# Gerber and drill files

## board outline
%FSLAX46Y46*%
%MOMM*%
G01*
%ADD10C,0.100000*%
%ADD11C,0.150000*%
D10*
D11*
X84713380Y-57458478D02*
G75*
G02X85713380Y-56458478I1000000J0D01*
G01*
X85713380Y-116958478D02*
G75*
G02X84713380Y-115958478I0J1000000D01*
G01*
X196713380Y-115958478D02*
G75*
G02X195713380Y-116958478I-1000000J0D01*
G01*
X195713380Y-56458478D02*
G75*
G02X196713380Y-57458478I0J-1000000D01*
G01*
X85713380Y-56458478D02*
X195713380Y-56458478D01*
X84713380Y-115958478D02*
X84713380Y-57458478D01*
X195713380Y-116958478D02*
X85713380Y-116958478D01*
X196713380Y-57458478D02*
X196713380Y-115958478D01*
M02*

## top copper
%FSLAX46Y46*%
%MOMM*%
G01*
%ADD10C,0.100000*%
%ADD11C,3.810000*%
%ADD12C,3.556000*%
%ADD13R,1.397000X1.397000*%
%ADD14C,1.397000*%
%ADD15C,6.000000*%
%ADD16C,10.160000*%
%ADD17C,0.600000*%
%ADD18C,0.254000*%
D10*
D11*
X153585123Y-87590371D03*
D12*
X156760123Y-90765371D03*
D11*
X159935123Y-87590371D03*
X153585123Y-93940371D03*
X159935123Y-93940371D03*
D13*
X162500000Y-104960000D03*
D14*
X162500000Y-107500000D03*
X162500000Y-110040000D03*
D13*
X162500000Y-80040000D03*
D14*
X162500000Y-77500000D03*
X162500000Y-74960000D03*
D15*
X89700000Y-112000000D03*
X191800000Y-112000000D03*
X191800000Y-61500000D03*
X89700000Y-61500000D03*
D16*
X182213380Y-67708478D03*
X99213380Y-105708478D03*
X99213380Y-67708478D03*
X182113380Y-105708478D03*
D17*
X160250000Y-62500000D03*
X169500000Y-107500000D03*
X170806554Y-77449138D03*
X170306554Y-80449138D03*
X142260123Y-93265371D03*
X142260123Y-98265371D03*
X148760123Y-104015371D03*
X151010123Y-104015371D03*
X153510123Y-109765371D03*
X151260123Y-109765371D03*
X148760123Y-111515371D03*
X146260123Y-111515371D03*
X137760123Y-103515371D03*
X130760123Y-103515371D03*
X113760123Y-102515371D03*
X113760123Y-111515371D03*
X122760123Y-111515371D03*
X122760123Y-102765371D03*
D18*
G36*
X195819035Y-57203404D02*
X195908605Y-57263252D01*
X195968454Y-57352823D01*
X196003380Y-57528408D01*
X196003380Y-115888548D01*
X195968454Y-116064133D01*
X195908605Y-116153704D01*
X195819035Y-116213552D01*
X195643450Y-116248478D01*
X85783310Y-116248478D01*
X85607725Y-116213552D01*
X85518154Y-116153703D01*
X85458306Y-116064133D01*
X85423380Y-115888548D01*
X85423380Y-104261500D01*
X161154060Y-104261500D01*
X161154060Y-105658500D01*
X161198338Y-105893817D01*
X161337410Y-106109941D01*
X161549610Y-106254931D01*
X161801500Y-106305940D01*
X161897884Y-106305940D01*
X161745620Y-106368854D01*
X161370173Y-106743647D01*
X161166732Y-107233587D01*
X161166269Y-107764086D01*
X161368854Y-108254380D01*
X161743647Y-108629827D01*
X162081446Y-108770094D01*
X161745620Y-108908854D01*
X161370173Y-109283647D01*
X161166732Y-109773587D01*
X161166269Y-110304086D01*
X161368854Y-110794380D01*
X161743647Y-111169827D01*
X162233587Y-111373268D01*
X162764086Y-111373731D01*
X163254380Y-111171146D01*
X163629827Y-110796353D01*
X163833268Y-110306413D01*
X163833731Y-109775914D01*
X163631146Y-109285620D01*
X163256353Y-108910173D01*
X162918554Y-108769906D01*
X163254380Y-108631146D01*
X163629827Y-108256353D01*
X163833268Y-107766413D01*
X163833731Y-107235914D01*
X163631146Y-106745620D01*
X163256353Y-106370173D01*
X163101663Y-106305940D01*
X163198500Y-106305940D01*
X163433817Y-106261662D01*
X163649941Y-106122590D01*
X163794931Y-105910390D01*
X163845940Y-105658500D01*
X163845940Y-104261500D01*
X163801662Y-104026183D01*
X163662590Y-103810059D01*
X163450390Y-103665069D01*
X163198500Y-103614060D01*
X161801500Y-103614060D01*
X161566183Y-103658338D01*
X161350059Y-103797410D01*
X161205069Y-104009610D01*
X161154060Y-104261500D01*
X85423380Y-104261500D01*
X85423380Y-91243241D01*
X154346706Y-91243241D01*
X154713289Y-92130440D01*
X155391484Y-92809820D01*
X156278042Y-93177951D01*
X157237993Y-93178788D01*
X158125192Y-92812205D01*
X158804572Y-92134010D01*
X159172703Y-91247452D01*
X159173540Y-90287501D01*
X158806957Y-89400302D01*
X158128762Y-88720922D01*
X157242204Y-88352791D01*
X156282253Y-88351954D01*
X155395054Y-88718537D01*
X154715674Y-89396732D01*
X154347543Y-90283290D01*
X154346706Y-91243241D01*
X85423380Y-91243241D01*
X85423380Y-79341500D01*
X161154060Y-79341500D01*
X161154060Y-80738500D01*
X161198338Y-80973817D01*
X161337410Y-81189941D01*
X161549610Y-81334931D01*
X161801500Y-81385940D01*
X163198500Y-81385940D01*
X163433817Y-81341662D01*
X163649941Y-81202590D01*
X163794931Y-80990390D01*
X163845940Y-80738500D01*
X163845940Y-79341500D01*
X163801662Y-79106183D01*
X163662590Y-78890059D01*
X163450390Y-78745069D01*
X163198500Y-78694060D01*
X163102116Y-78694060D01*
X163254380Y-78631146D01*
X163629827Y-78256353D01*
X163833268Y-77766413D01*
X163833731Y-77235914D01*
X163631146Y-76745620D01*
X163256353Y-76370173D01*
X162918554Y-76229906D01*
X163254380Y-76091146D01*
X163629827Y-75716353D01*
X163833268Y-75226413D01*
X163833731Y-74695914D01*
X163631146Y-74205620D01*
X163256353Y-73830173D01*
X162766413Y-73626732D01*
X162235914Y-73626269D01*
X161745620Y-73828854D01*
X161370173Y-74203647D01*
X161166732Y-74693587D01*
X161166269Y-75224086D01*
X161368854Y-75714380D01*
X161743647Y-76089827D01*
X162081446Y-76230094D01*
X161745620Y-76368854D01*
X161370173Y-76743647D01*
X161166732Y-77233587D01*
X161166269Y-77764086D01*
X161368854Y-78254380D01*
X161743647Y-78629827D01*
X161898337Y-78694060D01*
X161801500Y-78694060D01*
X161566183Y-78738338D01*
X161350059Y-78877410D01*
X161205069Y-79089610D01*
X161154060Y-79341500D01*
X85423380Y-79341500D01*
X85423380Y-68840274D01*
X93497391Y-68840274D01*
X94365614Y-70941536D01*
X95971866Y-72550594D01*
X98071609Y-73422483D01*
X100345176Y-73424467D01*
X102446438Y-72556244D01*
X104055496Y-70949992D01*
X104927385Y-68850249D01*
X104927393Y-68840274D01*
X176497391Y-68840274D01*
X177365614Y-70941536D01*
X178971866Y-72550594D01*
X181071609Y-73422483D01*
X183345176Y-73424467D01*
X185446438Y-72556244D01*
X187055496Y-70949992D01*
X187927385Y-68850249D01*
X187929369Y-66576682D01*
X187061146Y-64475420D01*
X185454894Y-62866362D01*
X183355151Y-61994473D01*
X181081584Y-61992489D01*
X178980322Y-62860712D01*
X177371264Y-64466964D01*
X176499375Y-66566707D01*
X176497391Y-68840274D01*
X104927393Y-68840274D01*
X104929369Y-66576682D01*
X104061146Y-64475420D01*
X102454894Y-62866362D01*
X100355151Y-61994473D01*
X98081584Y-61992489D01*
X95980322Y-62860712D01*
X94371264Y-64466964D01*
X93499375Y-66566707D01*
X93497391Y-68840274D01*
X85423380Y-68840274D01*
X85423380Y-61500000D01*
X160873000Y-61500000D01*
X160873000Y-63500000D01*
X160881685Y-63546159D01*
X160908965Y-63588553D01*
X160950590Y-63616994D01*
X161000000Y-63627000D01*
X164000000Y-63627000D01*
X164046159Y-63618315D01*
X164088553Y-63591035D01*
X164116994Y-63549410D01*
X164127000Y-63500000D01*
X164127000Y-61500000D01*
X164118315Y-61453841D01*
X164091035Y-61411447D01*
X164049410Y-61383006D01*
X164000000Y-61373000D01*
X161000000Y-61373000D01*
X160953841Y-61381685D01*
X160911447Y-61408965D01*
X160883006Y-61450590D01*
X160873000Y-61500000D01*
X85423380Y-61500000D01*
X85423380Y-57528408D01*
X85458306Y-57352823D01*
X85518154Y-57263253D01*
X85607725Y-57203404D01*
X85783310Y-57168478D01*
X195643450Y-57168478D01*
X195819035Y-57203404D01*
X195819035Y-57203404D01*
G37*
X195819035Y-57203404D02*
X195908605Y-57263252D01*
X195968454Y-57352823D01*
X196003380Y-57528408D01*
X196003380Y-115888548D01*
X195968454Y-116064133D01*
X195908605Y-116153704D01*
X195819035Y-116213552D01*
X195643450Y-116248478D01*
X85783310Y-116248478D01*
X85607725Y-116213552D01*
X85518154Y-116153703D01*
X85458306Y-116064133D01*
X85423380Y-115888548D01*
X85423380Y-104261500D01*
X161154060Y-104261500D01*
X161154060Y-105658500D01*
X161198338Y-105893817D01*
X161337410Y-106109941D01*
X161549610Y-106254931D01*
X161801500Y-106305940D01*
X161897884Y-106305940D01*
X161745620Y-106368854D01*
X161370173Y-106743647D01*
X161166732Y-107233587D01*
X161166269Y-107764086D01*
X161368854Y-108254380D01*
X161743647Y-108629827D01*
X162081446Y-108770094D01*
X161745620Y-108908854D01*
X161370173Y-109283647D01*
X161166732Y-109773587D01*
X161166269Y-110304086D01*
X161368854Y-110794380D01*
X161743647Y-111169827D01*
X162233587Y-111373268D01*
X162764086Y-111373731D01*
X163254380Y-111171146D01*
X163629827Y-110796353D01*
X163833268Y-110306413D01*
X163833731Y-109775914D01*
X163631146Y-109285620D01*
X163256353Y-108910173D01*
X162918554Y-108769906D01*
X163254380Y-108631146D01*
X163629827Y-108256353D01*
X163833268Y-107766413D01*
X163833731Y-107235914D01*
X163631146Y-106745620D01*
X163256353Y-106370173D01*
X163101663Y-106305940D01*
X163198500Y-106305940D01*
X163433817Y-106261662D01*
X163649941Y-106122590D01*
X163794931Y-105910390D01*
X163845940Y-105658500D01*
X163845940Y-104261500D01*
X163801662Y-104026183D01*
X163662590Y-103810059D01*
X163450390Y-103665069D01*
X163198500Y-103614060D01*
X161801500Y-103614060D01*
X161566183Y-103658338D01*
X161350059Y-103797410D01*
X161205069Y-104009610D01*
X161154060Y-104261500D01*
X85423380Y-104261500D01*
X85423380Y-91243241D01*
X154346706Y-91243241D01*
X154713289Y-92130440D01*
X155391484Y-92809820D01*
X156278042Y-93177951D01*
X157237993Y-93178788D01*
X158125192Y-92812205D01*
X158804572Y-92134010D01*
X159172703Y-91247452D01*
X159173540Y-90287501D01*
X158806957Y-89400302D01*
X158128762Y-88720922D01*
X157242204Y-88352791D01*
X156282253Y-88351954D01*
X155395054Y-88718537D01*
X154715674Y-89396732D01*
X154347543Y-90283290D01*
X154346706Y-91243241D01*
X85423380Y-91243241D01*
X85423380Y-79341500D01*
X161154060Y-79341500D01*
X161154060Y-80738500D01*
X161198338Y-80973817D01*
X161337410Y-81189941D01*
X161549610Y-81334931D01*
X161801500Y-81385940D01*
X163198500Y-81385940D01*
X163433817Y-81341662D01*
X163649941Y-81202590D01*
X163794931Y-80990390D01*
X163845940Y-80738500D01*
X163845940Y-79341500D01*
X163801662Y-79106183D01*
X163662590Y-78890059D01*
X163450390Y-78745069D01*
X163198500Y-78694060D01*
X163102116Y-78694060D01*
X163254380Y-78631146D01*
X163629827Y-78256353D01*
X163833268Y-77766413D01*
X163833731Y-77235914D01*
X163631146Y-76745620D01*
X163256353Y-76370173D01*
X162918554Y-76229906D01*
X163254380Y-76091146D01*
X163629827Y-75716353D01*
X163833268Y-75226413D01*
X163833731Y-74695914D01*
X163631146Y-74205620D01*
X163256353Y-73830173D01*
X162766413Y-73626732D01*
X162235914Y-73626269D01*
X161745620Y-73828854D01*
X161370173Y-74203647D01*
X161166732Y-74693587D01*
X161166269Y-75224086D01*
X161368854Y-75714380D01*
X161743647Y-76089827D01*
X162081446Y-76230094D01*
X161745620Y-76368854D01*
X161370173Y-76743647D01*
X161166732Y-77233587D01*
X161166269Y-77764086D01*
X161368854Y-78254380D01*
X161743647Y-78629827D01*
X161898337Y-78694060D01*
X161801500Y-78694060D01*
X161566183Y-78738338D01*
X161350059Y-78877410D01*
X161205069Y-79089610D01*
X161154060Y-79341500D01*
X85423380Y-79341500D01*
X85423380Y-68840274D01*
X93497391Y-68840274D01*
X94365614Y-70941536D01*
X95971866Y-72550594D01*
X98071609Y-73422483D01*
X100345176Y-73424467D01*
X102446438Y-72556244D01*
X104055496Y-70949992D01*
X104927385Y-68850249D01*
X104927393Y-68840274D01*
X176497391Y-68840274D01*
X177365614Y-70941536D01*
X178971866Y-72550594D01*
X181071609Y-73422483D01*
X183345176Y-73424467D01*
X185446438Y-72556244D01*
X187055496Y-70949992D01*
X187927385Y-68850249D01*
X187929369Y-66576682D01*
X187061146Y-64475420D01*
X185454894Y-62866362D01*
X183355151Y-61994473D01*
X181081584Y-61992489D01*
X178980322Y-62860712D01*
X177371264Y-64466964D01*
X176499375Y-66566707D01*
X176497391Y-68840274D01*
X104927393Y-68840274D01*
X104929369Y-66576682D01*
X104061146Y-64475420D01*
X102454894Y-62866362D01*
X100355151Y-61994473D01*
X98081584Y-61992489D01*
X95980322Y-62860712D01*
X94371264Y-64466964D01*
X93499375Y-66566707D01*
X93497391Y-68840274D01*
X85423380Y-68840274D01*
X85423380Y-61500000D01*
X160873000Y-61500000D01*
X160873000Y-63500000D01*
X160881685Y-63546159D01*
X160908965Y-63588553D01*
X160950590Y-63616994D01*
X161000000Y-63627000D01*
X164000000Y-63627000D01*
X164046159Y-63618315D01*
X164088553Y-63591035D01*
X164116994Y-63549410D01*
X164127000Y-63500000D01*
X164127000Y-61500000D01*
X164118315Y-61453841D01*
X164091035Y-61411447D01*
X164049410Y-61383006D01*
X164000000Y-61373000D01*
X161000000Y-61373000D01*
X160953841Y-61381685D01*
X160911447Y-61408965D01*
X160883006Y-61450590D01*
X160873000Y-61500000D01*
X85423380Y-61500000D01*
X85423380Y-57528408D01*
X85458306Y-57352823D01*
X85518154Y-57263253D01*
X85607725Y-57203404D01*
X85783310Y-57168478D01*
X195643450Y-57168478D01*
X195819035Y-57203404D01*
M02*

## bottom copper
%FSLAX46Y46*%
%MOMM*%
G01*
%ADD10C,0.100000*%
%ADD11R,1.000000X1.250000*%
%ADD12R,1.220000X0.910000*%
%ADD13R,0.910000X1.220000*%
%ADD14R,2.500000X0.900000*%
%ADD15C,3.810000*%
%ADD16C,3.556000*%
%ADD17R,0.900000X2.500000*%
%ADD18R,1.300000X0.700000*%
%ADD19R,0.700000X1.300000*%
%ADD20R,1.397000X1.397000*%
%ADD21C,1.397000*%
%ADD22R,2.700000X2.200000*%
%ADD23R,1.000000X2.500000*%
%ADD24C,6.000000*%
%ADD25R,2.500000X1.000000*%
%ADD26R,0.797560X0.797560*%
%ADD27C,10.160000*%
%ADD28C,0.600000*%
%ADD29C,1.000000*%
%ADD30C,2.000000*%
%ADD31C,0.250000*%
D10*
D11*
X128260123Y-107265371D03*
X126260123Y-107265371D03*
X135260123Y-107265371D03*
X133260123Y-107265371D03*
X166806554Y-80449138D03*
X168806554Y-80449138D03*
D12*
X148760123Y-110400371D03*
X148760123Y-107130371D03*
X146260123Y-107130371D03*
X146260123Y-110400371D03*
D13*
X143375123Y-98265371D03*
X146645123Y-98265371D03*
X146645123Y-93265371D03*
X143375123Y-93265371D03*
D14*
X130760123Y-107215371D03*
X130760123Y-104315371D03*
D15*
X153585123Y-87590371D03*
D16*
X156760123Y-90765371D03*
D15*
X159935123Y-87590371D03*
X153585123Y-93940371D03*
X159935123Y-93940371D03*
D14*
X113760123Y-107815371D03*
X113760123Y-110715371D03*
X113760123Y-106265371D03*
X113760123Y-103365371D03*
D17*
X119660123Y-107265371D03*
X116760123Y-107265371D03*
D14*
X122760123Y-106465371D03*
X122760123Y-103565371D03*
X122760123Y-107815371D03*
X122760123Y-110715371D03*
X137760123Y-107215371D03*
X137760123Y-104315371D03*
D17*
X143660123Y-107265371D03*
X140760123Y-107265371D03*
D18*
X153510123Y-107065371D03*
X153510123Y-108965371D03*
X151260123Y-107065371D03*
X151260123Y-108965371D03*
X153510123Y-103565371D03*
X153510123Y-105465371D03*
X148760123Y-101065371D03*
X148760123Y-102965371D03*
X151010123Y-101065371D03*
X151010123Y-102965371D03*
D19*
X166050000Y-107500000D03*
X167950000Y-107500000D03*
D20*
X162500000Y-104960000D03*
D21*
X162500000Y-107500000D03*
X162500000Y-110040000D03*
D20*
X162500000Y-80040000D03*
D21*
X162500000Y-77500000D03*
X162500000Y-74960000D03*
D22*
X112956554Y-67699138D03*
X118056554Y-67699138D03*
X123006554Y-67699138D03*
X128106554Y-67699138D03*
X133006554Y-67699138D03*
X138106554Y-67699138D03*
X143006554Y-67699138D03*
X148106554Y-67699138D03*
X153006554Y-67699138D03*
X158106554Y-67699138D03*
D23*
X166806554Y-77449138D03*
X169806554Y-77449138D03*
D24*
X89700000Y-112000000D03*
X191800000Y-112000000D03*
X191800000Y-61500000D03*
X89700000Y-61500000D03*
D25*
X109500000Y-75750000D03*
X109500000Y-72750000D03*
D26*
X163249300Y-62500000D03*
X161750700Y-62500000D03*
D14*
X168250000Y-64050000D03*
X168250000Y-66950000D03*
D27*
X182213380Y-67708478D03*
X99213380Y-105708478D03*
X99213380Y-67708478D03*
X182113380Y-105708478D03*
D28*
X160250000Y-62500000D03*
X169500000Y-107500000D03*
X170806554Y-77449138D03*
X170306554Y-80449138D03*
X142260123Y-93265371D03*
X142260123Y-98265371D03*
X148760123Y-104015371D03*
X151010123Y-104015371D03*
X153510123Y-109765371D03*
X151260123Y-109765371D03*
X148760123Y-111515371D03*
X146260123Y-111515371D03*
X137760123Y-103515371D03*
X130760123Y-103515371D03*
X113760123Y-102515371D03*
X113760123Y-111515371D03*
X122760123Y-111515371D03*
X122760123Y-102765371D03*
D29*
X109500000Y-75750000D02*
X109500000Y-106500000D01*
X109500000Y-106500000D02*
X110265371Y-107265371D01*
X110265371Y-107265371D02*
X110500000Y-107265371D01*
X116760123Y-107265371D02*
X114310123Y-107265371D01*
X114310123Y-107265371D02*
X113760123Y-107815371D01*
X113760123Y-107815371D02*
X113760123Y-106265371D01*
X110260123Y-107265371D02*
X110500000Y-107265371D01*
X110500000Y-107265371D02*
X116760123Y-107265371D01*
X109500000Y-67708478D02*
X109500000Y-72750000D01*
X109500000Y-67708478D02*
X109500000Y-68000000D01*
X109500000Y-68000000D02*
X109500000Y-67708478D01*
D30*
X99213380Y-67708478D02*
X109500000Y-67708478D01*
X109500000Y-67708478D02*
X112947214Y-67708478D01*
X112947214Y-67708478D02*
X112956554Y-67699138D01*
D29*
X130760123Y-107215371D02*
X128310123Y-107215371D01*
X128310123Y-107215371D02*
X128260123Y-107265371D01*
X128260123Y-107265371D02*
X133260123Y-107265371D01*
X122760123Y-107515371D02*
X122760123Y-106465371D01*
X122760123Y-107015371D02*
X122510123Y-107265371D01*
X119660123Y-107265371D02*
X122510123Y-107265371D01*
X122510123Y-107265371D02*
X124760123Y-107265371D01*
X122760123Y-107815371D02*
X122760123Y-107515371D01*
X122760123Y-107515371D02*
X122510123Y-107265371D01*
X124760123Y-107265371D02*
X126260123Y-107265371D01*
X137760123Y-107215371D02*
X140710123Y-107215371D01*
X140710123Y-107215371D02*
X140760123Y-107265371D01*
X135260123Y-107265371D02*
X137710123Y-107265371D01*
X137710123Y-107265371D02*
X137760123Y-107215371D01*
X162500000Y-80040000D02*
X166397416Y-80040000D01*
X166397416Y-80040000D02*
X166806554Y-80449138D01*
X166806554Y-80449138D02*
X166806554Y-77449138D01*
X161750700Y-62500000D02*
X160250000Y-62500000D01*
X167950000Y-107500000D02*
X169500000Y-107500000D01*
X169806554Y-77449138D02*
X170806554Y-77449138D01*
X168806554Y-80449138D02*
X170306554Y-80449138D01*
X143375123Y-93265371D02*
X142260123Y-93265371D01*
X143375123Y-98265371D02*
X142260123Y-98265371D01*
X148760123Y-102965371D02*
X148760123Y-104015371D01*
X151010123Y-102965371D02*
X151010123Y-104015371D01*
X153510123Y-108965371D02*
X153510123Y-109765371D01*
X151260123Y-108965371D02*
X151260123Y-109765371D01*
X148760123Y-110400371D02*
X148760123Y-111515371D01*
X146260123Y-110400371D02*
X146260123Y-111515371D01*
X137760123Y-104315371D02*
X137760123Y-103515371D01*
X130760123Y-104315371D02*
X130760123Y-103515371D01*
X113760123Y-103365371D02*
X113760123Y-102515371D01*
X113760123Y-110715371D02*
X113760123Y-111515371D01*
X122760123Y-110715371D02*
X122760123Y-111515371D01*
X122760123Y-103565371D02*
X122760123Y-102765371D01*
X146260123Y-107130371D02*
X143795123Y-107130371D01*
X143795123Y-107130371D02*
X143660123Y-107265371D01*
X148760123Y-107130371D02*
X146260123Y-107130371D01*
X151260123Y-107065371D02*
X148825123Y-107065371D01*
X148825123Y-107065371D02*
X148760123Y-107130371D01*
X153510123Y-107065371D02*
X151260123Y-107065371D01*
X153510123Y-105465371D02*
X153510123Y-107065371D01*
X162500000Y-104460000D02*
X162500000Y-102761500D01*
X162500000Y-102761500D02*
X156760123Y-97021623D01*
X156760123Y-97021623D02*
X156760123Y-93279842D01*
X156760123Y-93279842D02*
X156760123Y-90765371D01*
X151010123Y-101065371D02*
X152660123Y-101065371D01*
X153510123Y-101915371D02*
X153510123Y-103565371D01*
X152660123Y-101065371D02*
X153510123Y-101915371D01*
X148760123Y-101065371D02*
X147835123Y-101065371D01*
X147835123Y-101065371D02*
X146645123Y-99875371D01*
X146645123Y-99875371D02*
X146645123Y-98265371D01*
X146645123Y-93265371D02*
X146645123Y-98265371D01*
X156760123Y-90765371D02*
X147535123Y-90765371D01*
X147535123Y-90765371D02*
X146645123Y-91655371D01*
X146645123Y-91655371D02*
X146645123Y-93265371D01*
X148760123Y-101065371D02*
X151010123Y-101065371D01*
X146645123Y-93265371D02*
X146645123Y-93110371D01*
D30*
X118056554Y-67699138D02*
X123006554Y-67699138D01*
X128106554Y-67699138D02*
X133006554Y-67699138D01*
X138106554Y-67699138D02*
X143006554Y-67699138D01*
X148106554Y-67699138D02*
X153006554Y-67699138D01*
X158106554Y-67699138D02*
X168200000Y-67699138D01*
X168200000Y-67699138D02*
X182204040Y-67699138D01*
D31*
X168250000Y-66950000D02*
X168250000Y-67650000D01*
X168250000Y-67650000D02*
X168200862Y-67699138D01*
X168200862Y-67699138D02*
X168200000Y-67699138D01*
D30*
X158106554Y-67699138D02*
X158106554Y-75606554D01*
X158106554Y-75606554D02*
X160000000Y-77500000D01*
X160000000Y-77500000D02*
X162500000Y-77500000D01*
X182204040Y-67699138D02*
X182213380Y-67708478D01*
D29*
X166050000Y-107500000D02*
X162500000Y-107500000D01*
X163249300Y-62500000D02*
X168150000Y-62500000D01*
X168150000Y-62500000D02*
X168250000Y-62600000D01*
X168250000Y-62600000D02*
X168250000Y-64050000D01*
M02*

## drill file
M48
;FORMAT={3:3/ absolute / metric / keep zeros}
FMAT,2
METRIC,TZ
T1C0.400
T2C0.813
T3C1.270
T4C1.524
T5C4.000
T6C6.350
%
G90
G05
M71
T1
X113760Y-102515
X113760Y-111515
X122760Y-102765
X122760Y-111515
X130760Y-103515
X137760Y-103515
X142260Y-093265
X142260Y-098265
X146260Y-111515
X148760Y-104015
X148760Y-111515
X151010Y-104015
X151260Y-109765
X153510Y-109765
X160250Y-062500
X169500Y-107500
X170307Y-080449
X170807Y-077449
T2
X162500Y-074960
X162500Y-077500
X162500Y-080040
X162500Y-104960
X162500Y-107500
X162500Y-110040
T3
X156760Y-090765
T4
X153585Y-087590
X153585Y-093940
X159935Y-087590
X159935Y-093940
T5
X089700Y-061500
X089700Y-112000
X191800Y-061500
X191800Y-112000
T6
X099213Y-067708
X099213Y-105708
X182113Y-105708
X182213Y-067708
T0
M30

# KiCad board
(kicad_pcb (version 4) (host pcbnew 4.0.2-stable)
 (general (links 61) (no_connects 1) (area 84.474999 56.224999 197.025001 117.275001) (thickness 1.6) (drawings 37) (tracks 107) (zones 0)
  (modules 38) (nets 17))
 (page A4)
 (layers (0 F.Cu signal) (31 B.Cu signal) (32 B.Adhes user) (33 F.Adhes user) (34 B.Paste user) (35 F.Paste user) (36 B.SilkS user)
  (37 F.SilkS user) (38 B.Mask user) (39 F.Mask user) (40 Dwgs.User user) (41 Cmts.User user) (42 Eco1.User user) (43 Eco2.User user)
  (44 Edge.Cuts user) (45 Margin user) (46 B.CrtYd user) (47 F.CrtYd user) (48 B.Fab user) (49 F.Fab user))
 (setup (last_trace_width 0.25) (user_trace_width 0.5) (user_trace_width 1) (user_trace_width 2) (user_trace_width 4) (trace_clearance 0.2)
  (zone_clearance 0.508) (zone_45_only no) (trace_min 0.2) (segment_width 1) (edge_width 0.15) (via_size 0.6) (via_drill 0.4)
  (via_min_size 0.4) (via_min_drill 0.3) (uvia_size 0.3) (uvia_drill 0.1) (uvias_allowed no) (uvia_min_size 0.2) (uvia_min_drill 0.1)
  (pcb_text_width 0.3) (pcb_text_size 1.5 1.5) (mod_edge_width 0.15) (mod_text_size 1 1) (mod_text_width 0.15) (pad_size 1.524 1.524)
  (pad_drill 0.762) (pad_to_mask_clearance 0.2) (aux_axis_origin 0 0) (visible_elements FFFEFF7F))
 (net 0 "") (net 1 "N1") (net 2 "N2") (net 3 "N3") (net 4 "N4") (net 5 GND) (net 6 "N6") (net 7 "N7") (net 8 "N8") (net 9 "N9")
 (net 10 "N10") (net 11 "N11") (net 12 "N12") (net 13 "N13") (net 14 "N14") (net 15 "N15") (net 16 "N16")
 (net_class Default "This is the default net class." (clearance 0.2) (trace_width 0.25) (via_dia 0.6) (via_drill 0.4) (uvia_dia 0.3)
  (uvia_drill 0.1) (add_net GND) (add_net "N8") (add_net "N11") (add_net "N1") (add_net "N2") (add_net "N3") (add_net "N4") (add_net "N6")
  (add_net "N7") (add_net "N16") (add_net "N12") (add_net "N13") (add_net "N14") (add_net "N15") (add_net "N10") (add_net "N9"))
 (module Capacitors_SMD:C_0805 (layer B.Cu) (at 127.260123 107.265371 180)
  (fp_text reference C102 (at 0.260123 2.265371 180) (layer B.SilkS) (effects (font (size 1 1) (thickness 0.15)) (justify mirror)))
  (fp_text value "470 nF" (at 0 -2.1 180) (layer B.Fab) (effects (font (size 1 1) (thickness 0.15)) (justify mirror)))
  (pad 1 smd rect (at -1 0 180) (size 1 1.25) (layers B.Cu B.Paste B.Mask) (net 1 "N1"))
  (pad 2 smd rect (at 1 0 180) (size 1 1.25) (layers B.Cu B.Paste B.Mask) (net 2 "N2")))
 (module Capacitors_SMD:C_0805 (layer B.Cu) (at 134.260123 107.265371 180)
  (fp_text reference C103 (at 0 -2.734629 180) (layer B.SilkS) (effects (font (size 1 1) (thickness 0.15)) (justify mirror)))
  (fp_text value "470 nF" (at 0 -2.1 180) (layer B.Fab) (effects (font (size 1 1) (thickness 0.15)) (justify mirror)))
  (pad 1 smd rect (at -1 0 180) (size 1 1.25) (layers B.Cu B.Paste B.Mask) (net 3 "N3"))
  (pad 2 smd rect (at 1 0 180) (size 1 1.25) (layers B.Cu B.Paste B.Mask) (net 1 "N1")))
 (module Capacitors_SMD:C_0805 (layer B.Cu) (at 167.806554 80.449138)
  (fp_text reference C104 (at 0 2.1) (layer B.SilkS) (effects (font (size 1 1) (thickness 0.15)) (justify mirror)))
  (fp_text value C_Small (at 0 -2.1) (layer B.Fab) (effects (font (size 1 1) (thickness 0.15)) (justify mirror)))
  (pad 1 smd rect (at -1 0) (size 1 1.25) (layers B.Cu B.Paste B.Mask) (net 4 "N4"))
  (pad 2 smd rect (at 1 0) (size 1 1.25) (layers B.Cu B.Paste B.Mask) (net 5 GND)))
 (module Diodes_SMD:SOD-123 (layer B.Cu) (at 148.760123 108.765371 90)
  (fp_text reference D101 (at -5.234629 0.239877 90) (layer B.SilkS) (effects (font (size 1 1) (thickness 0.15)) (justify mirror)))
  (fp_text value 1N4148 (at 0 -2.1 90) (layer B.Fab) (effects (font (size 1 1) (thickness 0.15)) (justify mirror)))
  (pad 1 smd rect (at -1.635 0 90) (size 0.91 1.22) (layers B.Cu B.Paste B.Mask) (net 5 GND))
  (pad 2 smd rect (at 1.635 0 90) (size 0.91 1.22) (layers B.Cu B.Paste B.Mask) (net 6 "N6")))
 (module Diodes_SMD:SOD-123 (layer B.Cu) (at 146.260123 108.765371 270)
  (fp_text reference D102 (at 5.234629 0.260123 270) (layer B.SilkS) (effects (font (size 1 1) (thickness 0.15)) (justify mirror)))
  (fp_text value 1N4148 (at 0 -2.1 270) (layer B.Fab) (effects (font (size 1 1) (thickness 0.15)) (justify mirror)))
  (pad 1 smd rect (at -1.635 0 270) (size 0.91 1.22) (layers B.Cu B.Paste B.Mask) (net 6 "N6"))
  (pad 2 smd rect (at 1.635 0 270) (size 0.91 1.22) (layers B.Cu B.Paste B.Mask) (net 5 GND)))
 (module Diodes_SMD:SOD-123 (layer B.Cu) (at 145.010123 98.265371)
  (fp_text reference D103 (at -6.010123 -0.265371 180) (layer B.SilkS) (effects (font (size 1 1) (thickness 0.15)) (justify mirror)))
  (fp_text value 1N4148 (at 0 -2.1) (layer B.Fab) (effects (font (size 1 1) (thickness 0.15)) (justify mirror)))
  (pad 1 smd rect (at -1.635 0) (size 0.91 1.22) (layers B.Cu B.Paste B.Mask) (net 5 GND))
  (pad 2 smd rect (at 1.635 0) (size 0.91 1.22) (layers B.Cu B.Paste B.Mask) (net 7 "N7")))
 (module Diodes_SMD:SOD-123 (layer B.Cu) (at 145.010123 93.265371 180)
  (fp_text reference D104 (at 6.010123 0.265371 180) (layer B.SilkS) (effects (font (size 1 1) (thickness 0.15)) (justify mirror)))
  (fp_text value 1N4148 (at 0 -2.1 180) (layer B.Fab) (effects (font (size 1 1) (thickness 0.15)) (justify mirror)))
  (pad 1 smd rect (at -1.635 0 180) (size 0.91 1.22) (layers B.Cu B.Paste B.Mask) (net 7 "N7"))
  (pad 2 smd rect (at 1.635 0 180) (size 0.91 1.22) (layers B.Cu B.Paste B.Mask) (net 5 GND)))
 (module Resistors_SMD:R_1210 (layer B.Cu) (at 130.760123 105.765371 90)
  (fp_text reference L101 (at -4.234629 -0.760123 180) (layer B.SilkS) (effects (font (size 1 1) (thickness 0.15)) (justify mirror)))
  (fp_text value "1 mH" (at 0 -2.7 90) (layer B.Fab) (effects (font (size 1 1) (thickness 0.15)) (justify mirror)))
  (pad 1 smd rect (at -1.45 0 90) (size 0.9 2.5) (layers B.Cu B.Paste B.Mask) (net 1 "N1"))
  (pad 2 smd rect (at 1.45 0 90) (size 0.9 2.5) (layers B.Cu B.Paste B.Mask) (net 5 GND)))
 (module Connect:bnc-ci (layer F.Cu) (at 156.760123 90.765371)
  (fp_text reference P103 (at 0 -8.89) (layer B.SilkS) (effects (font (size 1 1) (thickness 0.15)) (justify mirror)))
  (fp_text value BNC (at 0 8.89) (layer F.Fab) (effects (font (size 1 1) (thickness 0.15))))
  (pad 2 thru_hole circle (at -3.175 -3.175) (size 3.81 3.81) (drill 1.524) (layers *.Cu *.Mask F.SilkS) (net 5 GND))
  (pad 1 thru_hole circle (at 0 0) (size 3.556 3.556) (drill 1.27) (layers *.Cu *.Mask F.SilkS) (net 7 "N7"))
  (pad 2 thru_hole circle (at 3.175 -3.175) (size 3.81 3.81) (drill 1.524) (layers *.Cu *.Mask F.SilkS) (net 5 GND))
  (pad 2 thru_hole circle (at -3.175 3.175) (size 3.81 3.81) (drill 1.524) (layers *.Cu *.Mask F.SilkS) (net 5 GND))
  (pad 2 thru_hole circle (at 3.175 3.175) (size 3.81 3.81) (drill 1.524) (layers *.Cu *.Mask F.SilkS) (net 5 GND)))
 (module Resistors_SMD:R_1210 (layer B.Cu) (at 113.760123 109.265371 270)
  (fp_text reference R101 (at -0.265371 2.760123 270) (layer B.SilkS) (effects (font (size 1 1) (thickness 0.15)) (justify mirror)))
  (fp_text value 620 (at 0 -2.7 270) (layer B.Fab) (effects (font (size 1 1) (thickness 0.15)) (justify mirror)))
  (pad 1 smd rect (at -1.45 0 270) (size 0.9 2.5) (layers B.Cu B.Paste B.Mask) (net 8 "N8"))
  (pad 2 smd rect (at 1.45 0 270) (size 0.9 2.5) (layers B.Cu B.Paste B.Mask) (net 5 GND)))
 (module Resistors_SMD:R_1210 (layer B.Cu) (at 113.760123 104.815371 90)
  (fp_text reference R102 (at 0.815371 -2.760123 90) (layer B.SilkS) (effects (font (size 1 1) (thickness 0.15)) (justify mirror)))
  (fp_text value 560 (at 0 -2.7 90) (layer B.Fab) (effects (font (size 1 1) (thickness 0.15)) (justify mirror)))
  (pad 1 smd rect (at -1.45 0 90) (size 0.9 2.5) (layers B.Cu B.Paste B.Mask) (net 8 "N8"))
  (pad 2 smd rect (at 1.45 0 90) (size 0.9 2.5) (layers B.Cu B.Paste B.Mask) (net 5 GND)))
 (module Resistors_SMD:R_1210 (layer B.Cu) (at 118.210123 107.265371 180)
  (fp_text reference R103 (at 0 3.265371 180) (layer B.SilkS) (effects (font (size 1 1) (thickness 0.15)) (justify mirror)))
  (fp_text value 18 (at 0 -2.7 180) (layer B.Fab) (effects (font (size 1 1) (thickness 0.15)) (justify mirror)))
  (pad 1 smd rect (at -1.45 0 180) (size 0.9 2.5) (layers B.Cu B.Paste B.Mask) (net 2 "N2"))
  (pad 2 smd rect (at 1.45 0 180) (size 0.9 2.5) (layers B.Cu B.Paste B.Mask) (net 8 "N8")))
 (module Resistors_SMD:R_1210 (layer B.Cu) (at 122.760123 105.015371 90)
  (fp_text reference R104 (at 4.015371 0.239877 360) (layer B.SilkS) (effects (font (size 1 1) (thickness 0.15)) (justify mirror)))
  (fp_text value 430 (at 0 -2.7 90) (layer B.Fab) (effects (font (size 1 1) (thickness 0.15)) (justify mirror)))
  (pad 1 smd rect (at -1.45 0 90) (size 0.9 2.5) (layers B.Cu B.Paste B.Mask) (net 2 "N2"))
  (pad 2 smd rect (at 1.45 0 90) (size 0.9 2.5) (layers B.Cu B.Paste B.Mask) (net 5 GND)))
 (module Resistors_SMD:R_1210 (layer B.Cu) (at 122.760123 109.265371 270)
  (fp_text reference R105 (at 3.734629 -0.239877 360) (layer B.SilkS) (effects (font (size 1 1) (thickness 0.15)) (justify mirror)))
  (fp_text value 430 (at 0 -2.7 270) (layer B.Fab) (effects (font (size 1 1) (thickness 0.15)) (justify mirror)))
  (pad 1 smd rect (at -1.45 0 270) (size 0.9 2.5) (layers B.Cu B.Paste B.Mask) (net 2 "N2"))
  (pad 2 smd rect (at 1.45 0 270) (size 0.9 2.5) (layers B.Cu B.Paste B.Mask) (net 5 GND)))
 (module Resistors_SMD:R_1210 (layer B.Cu) (at 137.760123 105.765371 90)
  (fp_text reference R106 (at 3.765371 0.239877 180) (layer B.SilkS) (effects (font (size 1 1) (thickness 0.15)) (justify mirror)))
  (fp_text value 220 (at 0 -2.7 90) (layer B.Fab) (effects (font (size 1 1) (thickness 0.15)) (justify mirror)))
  (pad 1 smd rect (at -1.45 0 90) (size 0.9 2.5) (layers B.Cu B.Paste B.Mask) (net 3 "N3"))
  (pad 2 smd rect (at 1.45 0 90) (size 0.9 2.5) (layers B.Cu B.Paste B.Mask) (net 5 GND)))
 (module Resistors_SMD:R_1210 (layer B.Cu) (at 142.210123 107.265371 180)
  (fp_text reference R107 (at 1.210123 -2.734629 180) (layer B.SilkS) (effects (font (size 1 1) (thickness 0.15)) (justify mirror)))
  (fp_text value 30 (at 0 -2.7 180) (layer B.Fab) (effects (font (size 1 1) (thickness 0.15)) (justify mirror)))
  (pad 1 smd rect (at -1.45 0 180) (size 0.9 2.5) (layers B.Cu B.Paste B.Mask) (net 6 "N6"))
  (pad 2 smd rect (at 1.45 0 180) (size 0.9 2.5) (layers B.Cu B.Paste B.Mask) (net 3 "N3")))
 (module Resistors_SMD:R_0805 (layer B.Cu) (at 153.510123 108.015371 270)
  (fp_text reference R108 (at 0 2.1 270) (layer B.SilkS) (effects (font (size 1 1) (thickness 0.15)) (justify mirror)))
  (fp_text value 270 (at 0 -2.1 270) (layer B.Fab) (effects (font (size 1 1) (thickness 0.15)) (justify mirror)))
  (pad 1 smd rect (at -0.95 0 270) (size 0.7 1.3) (layers B.Cu B.Paste B.Mask) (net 6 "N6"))
  (pad 2 smd rect (at 0.95 0 270) (size 0.7 1.3) (layers B.Cu B.Paste B.Mask) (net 5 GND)))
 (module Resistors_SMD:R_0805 (layer B.Cu) (at 151.260123 108.015371 270)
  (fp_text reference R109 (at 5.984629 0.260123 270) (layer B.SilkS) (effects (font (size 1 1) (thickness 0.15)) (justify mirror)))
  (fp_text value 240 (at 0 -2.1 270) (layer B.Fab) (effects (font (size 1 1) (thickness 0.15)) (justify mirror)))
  (pad 1 smd rect (at -0.95 0 270) (size 0.7 1.3) (layers B.Cu B.Paste B.Mask) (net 6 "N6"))
  (pad 2 smd rect (at 0.95 0 270) (size 0.7 1.3) (layers B.Cu B.Paste B.Mask) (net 5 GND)))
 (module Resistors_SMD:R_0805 (layer B.Cu) (at 153.510123 104.515371 270)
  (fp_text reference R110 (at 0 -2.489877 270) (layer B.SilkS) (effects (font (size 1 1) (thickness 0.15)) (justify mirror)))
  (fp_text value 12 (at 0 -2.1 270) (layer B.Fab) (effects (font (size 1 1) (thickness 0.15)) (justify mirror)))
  (pad 1 smd rect (at -0.95 0 270) (size 0.7 1.3) (layers B.Cu B.Paste B.Mask) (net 7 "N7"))
  (pad 2 smd rect (at 0.95 0 270) (size 0.7 1.3) (layers B.Cu B.Paste B.Mask) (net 6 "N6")))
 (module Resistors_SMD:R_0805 (layer B.Cu) (at 148.760123 102.015371 270)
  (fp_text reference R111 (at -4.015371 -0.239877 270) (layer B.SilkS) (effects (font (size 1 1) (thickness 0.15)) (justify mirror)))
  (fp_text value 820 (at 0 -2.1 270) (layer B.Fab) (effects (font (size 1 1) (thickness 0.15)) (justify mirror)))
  (pad 1 smd rect (at -0.95 0 270) (size 0.7 1.3) (layers B.Cu B.Paste B.Mask) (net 7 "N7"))
  (pad 2 smd rect (at 0.95 0 270) (size 0.7 1.3) (layers B.Cu B.Paste B.Mask) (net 5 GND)))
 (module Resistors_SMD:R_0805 (layer B.Cu) (at 151.010123 102.015371 270)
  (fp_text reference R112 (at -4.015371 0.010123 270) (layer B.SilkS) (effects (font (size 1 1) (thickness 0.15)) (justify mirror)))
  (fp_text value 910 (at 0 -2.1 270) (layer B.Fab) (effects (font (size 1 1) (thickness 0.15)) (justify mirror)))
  (pad 1 smd rect (at -0.95 0 270) (size 0.7 1.3) (layers B.Cu B.Paste B.Mask) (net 7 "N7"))
  (pad 2 smd rect (at 0.95 0 270) (size 0.7 1.3) (layers B.Cu B.Paste B.Mask) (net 5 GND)))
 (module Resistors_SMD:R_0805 (layer B.Cu) (at 167 107.5)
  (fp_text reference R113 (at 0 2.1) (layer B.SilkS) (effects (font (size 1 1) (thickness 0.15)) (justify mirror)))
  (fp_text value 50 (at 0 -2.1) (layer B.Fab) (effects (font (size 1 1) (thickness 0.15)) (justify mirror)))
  (pad 1 smd rect (at -0.95 0) (size 0.7 1.3) (layers B.Cu B.Paste B.Mask) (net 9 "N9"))
  (pad 2 smd rect (at 0.95 0) (size 0.7 1.3) (layers B.Cu B.Paste B.Mask) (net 5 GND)))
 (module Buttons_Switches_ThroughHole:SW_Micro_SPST (layer F.Cu) (at 162.5 107.5 270)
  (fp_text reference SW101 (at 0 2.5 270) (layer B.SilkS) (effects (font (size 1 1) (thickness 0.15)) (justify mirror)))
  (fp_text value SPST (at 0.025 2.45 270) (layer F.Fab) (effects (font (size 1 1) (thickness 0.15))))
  (pad 1 thru_hole rect (at -2.54 0 270) (size 1.397 1.397) (drill 0.8128) (layers *.Cu *.Mask F.SilkS) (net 7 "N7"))
  (pad 2 thru_hole circle (at 0 0 270) (size 1.397 1.397) (drill 0.8128) (layers *.Cu *.Mask F.SilkS) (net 9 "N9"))
  (pad 3 thru_hole circle (at 2.54 0 270) (size 1.397 1.397) (drill 0.8128) (layers *.Cu *.Mask F.SilkS)))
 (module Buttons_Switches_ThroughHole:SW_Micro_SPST (layer F.Cu) (at 162.5 77.5 90)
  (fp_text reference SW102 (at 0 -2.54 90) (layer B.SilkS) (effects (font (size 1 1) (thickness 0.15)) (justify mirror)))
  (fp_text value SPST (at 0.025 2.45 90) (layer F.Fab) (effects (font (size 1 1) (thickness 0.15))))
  (pad 1 thru_hole rect (at -2.54 0 90) (size 1.397 1.397) (drill 0.8128) (layers *.Cu *.Mask F.SilkS) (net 4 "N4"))
  (pad 2 thru_hole circle (at 0 0 90) (size 1.397 1.397) (drill 0.8128) (layers *.Cu *.Mask F.SilkS) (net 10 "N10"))
  (pad 3 thru_hole circle (at 2.54 0 90) (size 1.397 1.397) (drill 0.8128) (layers *.Cu *.Mask F.SilkS)))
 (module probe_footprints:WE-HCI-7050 (layer B.Cu) (at 115.506554 67.699138)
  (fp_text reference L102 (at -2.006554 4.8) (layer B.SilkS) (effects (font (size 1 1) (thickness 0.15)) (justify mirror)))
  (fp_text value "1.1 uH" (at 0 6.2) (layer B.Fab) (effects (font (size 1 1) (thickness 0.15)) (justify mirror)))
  (pad 1 smd rect (at -2.55 0) (size 2.7 2.2) (layers B.Cu B.Paste B.Mask) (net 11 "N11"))
  (pad 2 smd rect (at 2.55 0) (size 2.7 2.2) (layers B.Cu B.Paste B.Mask) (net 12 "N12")))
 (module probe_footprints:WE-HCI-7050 (layer B.Cu) (at 125.556554 67.699138)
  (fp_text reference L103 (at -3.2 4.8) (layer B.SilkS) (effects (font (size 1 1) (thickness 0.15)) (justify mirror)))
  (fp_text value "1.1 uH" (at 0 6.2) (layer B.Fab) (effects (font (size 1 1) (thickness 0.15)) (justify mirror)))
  (pad 1 smd rect (at -2.55 0) (size 2.7 2.2) (layers B.Cu B.Paste B.Mask) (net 12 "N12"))
  (pad 2 smd rect (at 2.55 0) (size 2.7 2.2) (layers B.Cu B.Paste B.Mask) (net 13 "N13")))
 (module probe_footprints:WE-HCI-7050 (layer B.Cu) (at 135.556554 67.699138)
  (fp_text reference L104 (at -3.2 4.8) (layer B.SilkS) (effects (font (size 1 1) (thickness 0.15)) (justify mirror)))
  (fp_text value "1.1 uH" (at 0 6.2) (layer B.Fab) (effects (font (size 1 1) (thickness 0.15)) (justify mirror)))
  (pad 1 smd rect (at -2.55 0) (size 2.7 2.2) (layers B.Cu B.Paste B.Mask) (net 13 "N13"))
  (pad 2 smd rect (at 2.55 0) (size 2.7 2.2) (layers B.Cu B.Paste B.Mask) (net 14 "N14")))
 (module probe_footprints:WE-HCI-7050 (layer B.Cu) (at 145.556554 67.699138)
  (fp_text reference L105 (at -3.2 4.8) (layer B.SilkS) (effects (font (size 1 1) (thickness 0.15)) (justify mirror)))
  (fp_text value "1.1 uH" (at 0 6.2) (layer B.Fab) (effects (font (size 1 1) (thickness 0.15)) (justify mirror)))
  (pad 1 smd rect (at -2.55 0) (size 2.7 2.2) (layers B.Cu B.Paste B.Mask) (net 14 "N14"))
  (pad 2 smd rect (at 2.55 0) (size 2.7 2.2) (layers B.Cu B.Paste B.Mask) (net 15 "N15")))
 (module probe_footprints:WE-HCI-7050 (layer B.Cu) (at 155.556554 67.699138)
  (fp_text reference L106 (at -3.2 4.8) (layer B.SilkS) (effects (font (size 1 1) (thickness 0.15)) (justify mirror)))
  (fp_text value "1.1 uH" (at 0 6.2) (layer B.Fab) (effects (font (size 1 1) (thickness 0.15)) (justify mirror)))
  (pad 1 smd rect (at -2.55 0) (size 2.7 2.2) (layers B.Cu B.Paste B.Mask) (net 15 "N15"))
  (pad 2 smd rect (at 2.55 0) (size 2.7 2.2) (layers B.Cu B.Paste B.Mask) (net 10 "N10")))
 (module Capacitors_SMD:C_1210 (layer B.Cu) (at 168.306554 77.449138)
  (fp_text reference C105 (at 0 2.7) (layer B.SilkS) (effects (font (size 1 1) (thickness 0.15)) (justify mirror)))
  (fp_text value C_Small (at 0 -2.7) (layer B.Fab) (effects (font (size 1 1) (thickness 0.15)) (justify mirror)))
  (pad 1 smd rect (at -1.5 0) (size 1 2.5) (layers B.Cu B.Paste B.Mask) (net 4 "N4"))
  (pad 2 smd rect (at 1.5 0) (size 1 2.5) (layers B.Cu B.Paste B.Mask) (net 5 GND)))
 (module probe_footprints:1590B (layer B.Cu) (at 140.75 86.75 180)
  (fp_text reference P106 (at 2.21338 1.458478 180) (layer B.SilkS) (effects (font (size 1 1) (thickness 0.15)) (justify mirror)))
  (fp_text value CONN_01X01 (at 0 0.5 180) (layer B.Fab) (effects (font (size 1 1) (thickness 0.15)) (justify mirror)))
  (pad 1 thru_hole circle (at 51.05 -25.25 180) (size 6 6) (drill 4) (layers *.Cu *.Mask B.SilkS) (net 5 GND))
  (pad 1 thru_hole circle (at -51.05 -25.25 180) (size 6 6) (drill 4) (layers *.Cu *.Mask B.SilkS) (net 5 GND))
  (pad 1 thru_hole circle (at -51.05 25.25 180) (size 6 6) (drill 4) (layers *.Cu *.Mask B.SilkS) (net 5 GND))
  (pad 1 thru_hole circle (at 51.05 25.25 180) (size 6 6) (drill 4) (layers *.Cu *.Mask B.SilkS) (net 5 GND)))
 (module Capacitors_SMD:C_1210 (layer B.Cu) (at 109.5 74.25 90)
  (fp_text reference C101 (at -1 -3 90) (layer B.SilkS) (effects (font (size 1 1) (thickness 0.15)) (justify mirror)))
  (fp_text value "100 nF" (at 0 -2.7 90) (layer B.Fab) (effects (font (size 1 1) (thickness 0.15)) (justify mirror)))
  (pad 1 smd rect (at -1.5 0 90) (size 1 2.5) (layers B.Cu B.Paste B.Mask) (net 8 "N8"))
  (pad 2 smd rect (at 1.5 0 90) (size 1 2.5) (layers B.Cu B.Paste B.Mask) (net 11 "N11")))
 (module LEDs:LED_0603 (layer B.Cu) (at 162.5 62.5)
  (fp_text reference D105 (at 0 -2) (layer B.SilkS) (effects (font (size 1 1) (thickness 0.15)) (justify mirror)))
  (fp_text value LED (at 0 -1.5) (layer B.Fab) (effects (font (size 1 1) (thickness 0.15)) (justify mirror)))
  (pad 2 smd rect (at 0.7493 0 180) (size 0.79756 0.79756) (layers B.Cu B.Paste B.Mask) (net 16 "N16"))
  (pad 1 smd rect (at -0.7493 0 180) (size 0.79756 0.79756) (layers B.Cu B.Paste B.Mask) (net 5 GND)))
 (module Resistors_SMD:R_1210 (layer B.Cu) (at 168.25 65.5 270)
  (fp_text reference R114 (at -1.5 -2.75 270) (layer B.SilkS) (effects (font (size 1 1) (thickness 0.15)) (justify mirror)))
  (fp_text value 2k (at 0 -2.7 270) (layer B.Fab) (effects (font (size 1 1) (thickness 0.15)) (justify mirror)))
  (pad 1 smd rect (at -1.45 0 270) (size 0.9 2.5) (layers B.Cu B.Paste B.Mask) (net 16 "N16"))
  (pad 2 smd rect (at 1.45 0 270) (size 0.9 2.5) (layers B.Cu B.Paste B.Mask) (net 10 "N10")))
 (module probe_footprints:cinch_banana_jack (layer F.Cu) (at 182.21338 67.708478 270)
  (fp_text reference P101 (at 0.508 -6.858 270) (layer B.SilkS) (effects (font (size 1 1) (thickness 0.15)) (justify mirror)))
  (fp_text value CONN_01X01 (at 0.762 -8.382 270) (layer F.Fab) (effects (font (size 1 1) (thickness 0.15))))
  (pad 1 thru_hole circle (at 0 0 270) (size 10.16 10.16) (drill 6.35) (layers *.Cu *.Mask F.SilkS) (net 10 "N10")))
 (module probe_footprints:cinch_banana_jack (layer F.Cu) (at 99.21338 105.708478 270)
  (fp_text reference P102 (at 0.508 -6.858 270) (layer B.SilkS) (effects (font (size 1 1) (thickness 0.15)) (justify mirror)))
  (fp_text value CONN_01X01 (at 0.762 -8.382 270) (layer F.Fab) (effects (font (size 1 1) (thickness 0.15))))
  (pad 1 thru_hole circle (at 0 0 270) (size 10.16 10.16) (drill 6.35) (layers *.Cu *.Mask F.SilkS) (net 5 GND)))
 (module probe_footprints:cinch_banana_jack (layer F.Cu) (at 99.21338 67.708478 180)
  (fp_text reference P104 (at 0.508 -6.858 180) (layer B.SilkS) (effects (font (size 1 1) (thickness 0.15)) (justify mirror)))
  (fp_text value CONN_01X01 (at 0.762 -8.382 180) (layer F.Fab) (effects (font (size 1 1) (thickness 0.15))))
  (pad 1 thru_hole circle (at 0 0 180) (size 10.16 10.16) (drill 6.35) (layers *.Cu *.Mask F.SilkS) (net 11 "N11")))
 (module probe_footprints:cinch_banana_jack (layer F.Cu) (at 182.11338 105.708478 180)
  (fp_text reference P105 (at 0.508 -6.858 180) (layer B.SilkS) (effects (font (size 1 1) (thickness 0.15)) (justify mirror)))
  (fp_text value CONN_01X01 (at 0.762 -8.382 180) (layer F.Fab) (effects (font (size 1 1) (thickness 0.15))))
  (pad 1 thru_hole circle (at 0 0 180) (size 10.16 10.16) (drill 6.35) (layers *.Cu *.Mask F.SilkS) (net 5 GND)))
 (gr_arc (start 85.71338 57.458478) (end 85.71338 56.458478) (angle -90) (layer Edge.Cuts) (width 0.15))
 (gr_arc (start 85.71338 115.958478) (end 84.71338 115.958478) (angle -90) (layer Edge.Cuts) (width 0.15))
 (gr_arc (start 195.71338 115.958478) (end 195.71338 116.958478) (angle -90) (layer Edge.Cuts) (width 0.15))
 (gr_arc (start 195.71338 57.458478) (end 196.71338 57.458478) (angle -90) (layer Edge.Cuts) (width 0.15))
 (gr_line (start 85.71338 56.458478) (end 195.71338 56.458478) (layer Edge.Cuts) (width 0.15))
 (gr_line (start 84.71338 115.958478) (end 84.71338 57.458478) (layer Edge.Cuts) (width 0.15))
 (gr_line (start 195.71338 116.958478) (end 85.71338 116.958478) (layer Edge.Cuts) (width 0.15))
 (gr_line (start 196.71338 57.458478) (end 196.71338 115.958478) (layer Edge.Cuts) (width 0.15))
 (segment (start 109.5 75.75) (end 109.5 106.5) (width 1) (layer B.Cu) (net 8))
 (segment (start 109.5 106.5) (end 110.265371 107.265371) (width 1) (layer B.Cu) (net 8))
 (segment (start 110.265371 107.265371) (end 110.5 107.265371) (width 1) (layer B.Cu) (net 8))
 (segment (start 116.760123 107.265371) (end 114.310123 107.265371) (width 1) (layer B.Cu) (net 8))
 (segment (start 114.310123 107.265371) (end 113.760123 107.815371) (width 1) (layer B.Cu) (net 8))
 (segment (start 113.760123 107.815371) (end 113.760123 106.265371) (width 1) (layer B.Cu) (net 8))
 (segment (start 110.260123 107.265371) (end 110.5 107.265371) (width 1) (layer B.Cu) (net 8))
 (segment (start 110.5 107.265371) (end 116.760123 107.265371) (width 1) (layer B.Cu) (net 8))
 (segment (start 109.5 67.708478) (end 109.5 72.75) (width 1) (layer B.Cu) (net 11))
 (segment (start 109.5 67.708478) (end 109.5 68) (width 1) (layer B.Cu) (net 11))
 (segment (start 109.5 68) (end 109.5 67.708478) (width 1) (layer B.Cu) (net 11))
 (segment (start 99.21338 67.708478) (end 109.5 67.708478) (width 2) (layer B.Cu) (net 11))
 (segment (start 109.5 67.708478) (end 112.947214 67.708478) (width 2) (layer B.Cu) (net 11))
 (segment (start 112.947214 67.708478) (end 112.956554 67.699138) (width 2) (layer B.Cu) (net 11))
 (segment (start 130.760123 107.215371) (end 128.310123 107.215371) (width 1) (layer B.Cu) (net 1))
 (segment (start 128.310123 107.215371) (end 128.260123 107.265371) (width 1) (layer B.Cu) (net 1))
 (segment (start 128.260123 107.265371) (end 133.260123 107.265371) (width 1) (layer B.Cu) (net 1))
 (segment (start 122.760123 107.515371) (end 122.760123 106.465371) (width 1) (layer B.Cu) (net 2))
 (segment (start 122.760123 107.015371) (end 122.510123 107.265371) (width 1) (layer B.Cu) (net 2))
 (segment (start 119.660123 107.265371) (end 122.510123 107.265371) (width 1) (layer B.Cu) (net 2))
 (segment (start 122.510123 107.265371) (end 124.760123 107.265371) (width 1) (layer B.Cu) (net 2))
 (segment (start 122.760123 107.815371) (end 122.760123 107.515371) (width 1) (layer B.Cu) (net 2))
 (segment (start 122.760123 107.515371) (end 122.510123 107.265371) (width 1) (layer B.Cu) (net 2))
 (segment (start 124.760123 107.265371) (end 126.260123 107.265371) (width 1) (layer B.Cu) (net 2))
 (segment (start 137.760123 107.215371) (end 140.710123 107.215371) (width 1) (layer B.Cu) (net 3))
 (segment (start 140.710123 107.215371) (end 140.760123 107.265371) (width 1) (layer B.Cu) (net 3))
 (segment (start 135.260123 107.265371) (end 137.710123 107.265371) (width 1) (layer B.Cu) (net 3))
 (segment (start 137.710123 107.265371) (end 137.760123 107.215371) (width 1) (layer B.Cu) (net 3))
 (segment (start 162.5 80.04) (end 166.397416 80.04) (width 1) (layer B.Cu) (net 4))
 (segment (start 166.397416 80.04) (end 166.806554 80.449138) (width 1) (layer B.Cu) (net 4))
 (segment (start 166.806554 80.449138) (end 166.806554 77.449138) (width 1) (layer B.Cu) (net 4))
 (via (at 160.25 62.5) (size 0.6) (drill 0.4) (layers F.Cu B.Cu) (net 5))
 (segment (start 161.7507 62.5) (end 160.25 62.5) (width 1) (layer B.Cu) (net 5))
 (segment (start 167.95 107.5) (end 169.5 107.5) (width 1) (layer B.Cu) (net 5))
 (via (at 169.5 107.5) (size 0.6) (drill 0.4) (layers F.Cu B.Cu) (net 5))
 (via (at 170.806554 77.449138) (size 0.6) (drill 0.4) (layers F.Cu B.Cu) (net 5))
 (segment (start 169.806554 77.449138) (end 170.806554 77.449138) (width 1) (layer B.Cu) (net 5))
 (via (at 170.306554 80.449138) (size 0.6) (drill 0.4) (layers F.Cu B.Cu) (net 5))
 (segment (start 168.806554 80.449138) (end 170.306554 80.449138) (width 1) (layer B.Cu) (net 5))
 (via (at 142.260123 93.265371) (size 0.6) (drill 0.4) (layers F.Cu B.Cu) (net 5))
 (segment (start 143.375123 93.265371) (end 142.260123 93.265371) (width 1) (layer B.Cu) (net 5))
 (via (at 142.260123 98.265371) (size 0.6) (drill 0.4) (layers F.Cu B.Cu) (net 5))
 (segment (start 143.375123 98.265371) (end 142.260123 98.265371) (width 1) (layer B.Cu) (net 5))
 (via (at 148.760123 104.015371) (size 0.6) (drill 0.4) (layers F.Cu B.Cu) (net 5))
 (segment (start 148.760123 102.965371) (end 148.760123 104.015371) (width 1) (layer B.Cu) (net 5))
 (via (at 151.010123 104.015371) (size 0.6) (drill 0.4) (layers F.Cu B.Cu) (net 5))
 (segment (start 151.010123 102.965371) (end 151.010123 104.015371) (width 1) (layer B.Cu) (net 5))
 (via (at 153.510123 109.765371) (size 0.6) (drill 0.4) (layers F.Cu B.Cu) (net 5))
 (segment (start 153.510123 108.965371) (end 153.510123 109.765371) (width 1) (layer B.Cu) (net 5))
 (via (at 151.260123 109.765371) (size 0.6) (drill 0.4) (layers F.Cu B.Cu) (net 5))
 (segment (start 151.260123 108.965371) (end 151.260123 109.765371) (width 1) (layer B.Cu) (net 5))
 (via (at 148.760123 111.515371) (size 0.6) (drill 0.4) (layers F.Cu B.Cu) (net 5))
 (segment (start 148.760123 110.400371) (end 148.760123 111.515371) (width 1) (layer B.Cu) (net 5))
 (via (at 146.260123 111.515371) (size 0.6) (drill 0.4) (layers F.Cu B.Cu) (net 5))
 (segment (start 146.260123 110.400371) (end 146.260123 111.515371) (width 1) (layer B.Cu) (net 5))
 (via (at 137.760123 103.515371) (size 0.6) (drill 0.4) (layers F.Cu B.Cu) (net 5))
 (segment (start 137.760123 104.315371) (end 137.760123 103.515371) (width 1) (layer B.Cu) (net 5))
 (segment (start 130.760123 104.315371) (end 130.760123 103.515371) (width 1) (layer B.Cu) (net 5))
 (via (at 130.760123 103.515371) (size 0.6) (drill 0.4) (layers F.Cu B.Cu) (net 5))
 (via (at 113.760123 102.515371) (size 0.6) (drill 0.4) (layers F.Cu B.Cu) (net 5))
 (segment (start 113.760123 103.365371) (end 113.760123 102.515371) (width 1) (layer B.Cu) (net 5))
 (via (at 113.760123 111.515371) (size 0.6) (drill 0.4) (layers F.Cu B.Cu) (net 5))
 (segment (start 113.760123 110.715371) (end 113.760123 111.515371) (width 1) (layer B.Cu) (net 5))
 (via (at 122.760123 111.515371) (size 0.6) (drill 0.4) (layers F.Cu B.Cu) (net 5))
 (segment (start 122.760123 110.715371) (end 122.760123 111.515371) (width 1) (layer B.Cu) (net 5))
 (via (at 122.760123 102.765371) (size 0.6) (drill 0.4) (layers F.Cu B.Cu) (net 5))
 (segment (start 122.760123 103.565371) (end 122.760123 102.765371) (width 1) (layer B.Cu) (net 5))
 (segment (start 146.260123 107.130371) (end 143.795123 107.130371) (width 1) (layer B.Cu) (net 6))
 (segment (start 143.795123 107.130371) (end 143.660123 107.265371) (width 1) (layer B.Cu) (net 6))
 (segment (start 148.760123 107.130371) (end 146.260123 107.130371) (width 1) (layer B.Cu) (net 6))
 (segment (start 151.260123 107.065371) (end 148.825123 107.065371) (width 1) (layer B.Cu) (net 6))
 (segment (start 148.825123 107.065371) (end 148.760123 107.130371) (width 1) (layer B.Cu) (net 6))
 (segment (start 153.510123 107.065371) (end 151.260123 107.065371) (width 1) (layer B.Cu) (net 6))
 (segment (start 153.510123 105.465371) (end 153.510123 107.065371) (width 1) (layer B.Cu) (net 6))
 (segment (start 162.5 104.46) (end 162.5 102.7615) (width 1) (layer B.Cu) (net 7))
 (segment (start 162.5 102.7615) (end 156.760123 97.021623) (width 1) (layer B.Cu) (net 7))
 (segment (start 156.760123 97.021623) (end 156.760123 93.279842) (width 1) (layer B.Cu) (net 7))
 (segment (start 156.760123 93.279842) (end 156.760123 90.765371) (width 1) (layer B.Cu) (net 7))
 (segment (start 151.010123 101.065371) (end 152.660123 101.065371) (width 1) (layer B.Cu) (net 7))
 (segment (start 153.510123 101.915371) (end 153.510123 103.565371) (width 1) (layer B.Cu) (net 7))
 (segment (start 152.660123 101.065371) (end 153.510123 101.915371) (width 1) (layer B.Cu) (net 7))
 (segment (start 148.760123 101.065371) (end 147.835123 101.065371) (width 1) (layer B.Cu) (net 7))
 (segment (start 147.835123 101.065371) (end 146.645123 99.875371) (width 1) (layer B.Cu) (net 7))
 (segment (start 146.645123 99.875371) (end 146.645123 98.265371) (width 1) (layer B.Cu) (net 7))
 (segment (start 146.645123 93.265371) (end 146.645123 98.265371) (width 1) (layer B.Cu) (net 7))
 (segment (start 156.760123 90.765371) (end 147.535123 90.765371) (width 1) (layer B.Cu) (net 7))
 (segment (start 147.535123 90.765371) (end 146.645123 91.655371) (width 1) (layer B.Cu) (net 7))
 (segment (start 146.645123 91.655371) (end 146.645123 93.265371) (width 1) (layer B.Cu) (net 7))
 (segment (start 148.760123 101.065371) (end 151.010123 101.065371) (width 1) (layer B.Cu) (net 7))
 (segment (start 146.645123 93.265371) (end 146.645123 93.110371) (width 1) (layer B.Cu) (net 7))
 (segment (start 118.056554 67.699138) (end 123.006554 67.699138) (width 2) (layer B.Cu) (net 12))
 (segment (start 128.106554 67.699138) (end 133.006554 67.699138) (width 2) (layer B.Cu) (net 13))
 (segment (start 138.106554 67.699138) (end 143.006554 67.699138) (width 2) (layer B.Cu) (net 14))
 (segment (start 148.106554 67.699138) (end 153.006554 67.699138) (width 2) (layer B.Cu) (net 15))
 (segment (start 158.106554 67.699138) (end 168.2 67.699138) (width 2) (layer B.Cu) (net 10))
 (segment (start 168.2 67.699138) (end 182.20404 67.699138) (width 2) (layer B.Cu) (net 10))
 (segment (start 168.25 66.95) (end 168.25 67.65) (width 0.25) (layer B.Cu) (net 10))
 (segment (start 168.25 67.65) (end 168.200862 67.699138) (width 0.25) (layer B.Cu) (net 10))
 (segment (start 168.200862 67.699138) (end 168.2 67.699138) (width 0.25) (layer B.Cu) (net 10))
 (segment (start 158.106554 67.699138) (end 158.106554 75.606554) (width 2) (layer B.Cu) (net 10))
 (segment (start 158.106554 75.606554) (end 160 77.5) (width 2) (layer B.Cu) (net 10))
 (segment (start 160 77.5) (end 162.5 77.5) (width 2) (layer B.Cu) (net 10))
 (segment (start 182.20404 67.699138) (end 182.21338 67.708478) (width 2) (layer B.Cu) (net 10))
 (segment (start 166.05 107.5) (end 162.5 107.5) (width 1) (layer B.Cu) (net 9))
 (segment (start 163.2493 62.5) (end 168.15 62.5) (width 1) (layer B.Cu) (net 16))
 (segment (start 168.15 62.5) (end 168.25 62.6) (width 1) (layer B.Cu) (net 16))
 (segment (start 168.25 62.6) (end 168.25 64.05) (width 1) (layer B.Cu) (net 16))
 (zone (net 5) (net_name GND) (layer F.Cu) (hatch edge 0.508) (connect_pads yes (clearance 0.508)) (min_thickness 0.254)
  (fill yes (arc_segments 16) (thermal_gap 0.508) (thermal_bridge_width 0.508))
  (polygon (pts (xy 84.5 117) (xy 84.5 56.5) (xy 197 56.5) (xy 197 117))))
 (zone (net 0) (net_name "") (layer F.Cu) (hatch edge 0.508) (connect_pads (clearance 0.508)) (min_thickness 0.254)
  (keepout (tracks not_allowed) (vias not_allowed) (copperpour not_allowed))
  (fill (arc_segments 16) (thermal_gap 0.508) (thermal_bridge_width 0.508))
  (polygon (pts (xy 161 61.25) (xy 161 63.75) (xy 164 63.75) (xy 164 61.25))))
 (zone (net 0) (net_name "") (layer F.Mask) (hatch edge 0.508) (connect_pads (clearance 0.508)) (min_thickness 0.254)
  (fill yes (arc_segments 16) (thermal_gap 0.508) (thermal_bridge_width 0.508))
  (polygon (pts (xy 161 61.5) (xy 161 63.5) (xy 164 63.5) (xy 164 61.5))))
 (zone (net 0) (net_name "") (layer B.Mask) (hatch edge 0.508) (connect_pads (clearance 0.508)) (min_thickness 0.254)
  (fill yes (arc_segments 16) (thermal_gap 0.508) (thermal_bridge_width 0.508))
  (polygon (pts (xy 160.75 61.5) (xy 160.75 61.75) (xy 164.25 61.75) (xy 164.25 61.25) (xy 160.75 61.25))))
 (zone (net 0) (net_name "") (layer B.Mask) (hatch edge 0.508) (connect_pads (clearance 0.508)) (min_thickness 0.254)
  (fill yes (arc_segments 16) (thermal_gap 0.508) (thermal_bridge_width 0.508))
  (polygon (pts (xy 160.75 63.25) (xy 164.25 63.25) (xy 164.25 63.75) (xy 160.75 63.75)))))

